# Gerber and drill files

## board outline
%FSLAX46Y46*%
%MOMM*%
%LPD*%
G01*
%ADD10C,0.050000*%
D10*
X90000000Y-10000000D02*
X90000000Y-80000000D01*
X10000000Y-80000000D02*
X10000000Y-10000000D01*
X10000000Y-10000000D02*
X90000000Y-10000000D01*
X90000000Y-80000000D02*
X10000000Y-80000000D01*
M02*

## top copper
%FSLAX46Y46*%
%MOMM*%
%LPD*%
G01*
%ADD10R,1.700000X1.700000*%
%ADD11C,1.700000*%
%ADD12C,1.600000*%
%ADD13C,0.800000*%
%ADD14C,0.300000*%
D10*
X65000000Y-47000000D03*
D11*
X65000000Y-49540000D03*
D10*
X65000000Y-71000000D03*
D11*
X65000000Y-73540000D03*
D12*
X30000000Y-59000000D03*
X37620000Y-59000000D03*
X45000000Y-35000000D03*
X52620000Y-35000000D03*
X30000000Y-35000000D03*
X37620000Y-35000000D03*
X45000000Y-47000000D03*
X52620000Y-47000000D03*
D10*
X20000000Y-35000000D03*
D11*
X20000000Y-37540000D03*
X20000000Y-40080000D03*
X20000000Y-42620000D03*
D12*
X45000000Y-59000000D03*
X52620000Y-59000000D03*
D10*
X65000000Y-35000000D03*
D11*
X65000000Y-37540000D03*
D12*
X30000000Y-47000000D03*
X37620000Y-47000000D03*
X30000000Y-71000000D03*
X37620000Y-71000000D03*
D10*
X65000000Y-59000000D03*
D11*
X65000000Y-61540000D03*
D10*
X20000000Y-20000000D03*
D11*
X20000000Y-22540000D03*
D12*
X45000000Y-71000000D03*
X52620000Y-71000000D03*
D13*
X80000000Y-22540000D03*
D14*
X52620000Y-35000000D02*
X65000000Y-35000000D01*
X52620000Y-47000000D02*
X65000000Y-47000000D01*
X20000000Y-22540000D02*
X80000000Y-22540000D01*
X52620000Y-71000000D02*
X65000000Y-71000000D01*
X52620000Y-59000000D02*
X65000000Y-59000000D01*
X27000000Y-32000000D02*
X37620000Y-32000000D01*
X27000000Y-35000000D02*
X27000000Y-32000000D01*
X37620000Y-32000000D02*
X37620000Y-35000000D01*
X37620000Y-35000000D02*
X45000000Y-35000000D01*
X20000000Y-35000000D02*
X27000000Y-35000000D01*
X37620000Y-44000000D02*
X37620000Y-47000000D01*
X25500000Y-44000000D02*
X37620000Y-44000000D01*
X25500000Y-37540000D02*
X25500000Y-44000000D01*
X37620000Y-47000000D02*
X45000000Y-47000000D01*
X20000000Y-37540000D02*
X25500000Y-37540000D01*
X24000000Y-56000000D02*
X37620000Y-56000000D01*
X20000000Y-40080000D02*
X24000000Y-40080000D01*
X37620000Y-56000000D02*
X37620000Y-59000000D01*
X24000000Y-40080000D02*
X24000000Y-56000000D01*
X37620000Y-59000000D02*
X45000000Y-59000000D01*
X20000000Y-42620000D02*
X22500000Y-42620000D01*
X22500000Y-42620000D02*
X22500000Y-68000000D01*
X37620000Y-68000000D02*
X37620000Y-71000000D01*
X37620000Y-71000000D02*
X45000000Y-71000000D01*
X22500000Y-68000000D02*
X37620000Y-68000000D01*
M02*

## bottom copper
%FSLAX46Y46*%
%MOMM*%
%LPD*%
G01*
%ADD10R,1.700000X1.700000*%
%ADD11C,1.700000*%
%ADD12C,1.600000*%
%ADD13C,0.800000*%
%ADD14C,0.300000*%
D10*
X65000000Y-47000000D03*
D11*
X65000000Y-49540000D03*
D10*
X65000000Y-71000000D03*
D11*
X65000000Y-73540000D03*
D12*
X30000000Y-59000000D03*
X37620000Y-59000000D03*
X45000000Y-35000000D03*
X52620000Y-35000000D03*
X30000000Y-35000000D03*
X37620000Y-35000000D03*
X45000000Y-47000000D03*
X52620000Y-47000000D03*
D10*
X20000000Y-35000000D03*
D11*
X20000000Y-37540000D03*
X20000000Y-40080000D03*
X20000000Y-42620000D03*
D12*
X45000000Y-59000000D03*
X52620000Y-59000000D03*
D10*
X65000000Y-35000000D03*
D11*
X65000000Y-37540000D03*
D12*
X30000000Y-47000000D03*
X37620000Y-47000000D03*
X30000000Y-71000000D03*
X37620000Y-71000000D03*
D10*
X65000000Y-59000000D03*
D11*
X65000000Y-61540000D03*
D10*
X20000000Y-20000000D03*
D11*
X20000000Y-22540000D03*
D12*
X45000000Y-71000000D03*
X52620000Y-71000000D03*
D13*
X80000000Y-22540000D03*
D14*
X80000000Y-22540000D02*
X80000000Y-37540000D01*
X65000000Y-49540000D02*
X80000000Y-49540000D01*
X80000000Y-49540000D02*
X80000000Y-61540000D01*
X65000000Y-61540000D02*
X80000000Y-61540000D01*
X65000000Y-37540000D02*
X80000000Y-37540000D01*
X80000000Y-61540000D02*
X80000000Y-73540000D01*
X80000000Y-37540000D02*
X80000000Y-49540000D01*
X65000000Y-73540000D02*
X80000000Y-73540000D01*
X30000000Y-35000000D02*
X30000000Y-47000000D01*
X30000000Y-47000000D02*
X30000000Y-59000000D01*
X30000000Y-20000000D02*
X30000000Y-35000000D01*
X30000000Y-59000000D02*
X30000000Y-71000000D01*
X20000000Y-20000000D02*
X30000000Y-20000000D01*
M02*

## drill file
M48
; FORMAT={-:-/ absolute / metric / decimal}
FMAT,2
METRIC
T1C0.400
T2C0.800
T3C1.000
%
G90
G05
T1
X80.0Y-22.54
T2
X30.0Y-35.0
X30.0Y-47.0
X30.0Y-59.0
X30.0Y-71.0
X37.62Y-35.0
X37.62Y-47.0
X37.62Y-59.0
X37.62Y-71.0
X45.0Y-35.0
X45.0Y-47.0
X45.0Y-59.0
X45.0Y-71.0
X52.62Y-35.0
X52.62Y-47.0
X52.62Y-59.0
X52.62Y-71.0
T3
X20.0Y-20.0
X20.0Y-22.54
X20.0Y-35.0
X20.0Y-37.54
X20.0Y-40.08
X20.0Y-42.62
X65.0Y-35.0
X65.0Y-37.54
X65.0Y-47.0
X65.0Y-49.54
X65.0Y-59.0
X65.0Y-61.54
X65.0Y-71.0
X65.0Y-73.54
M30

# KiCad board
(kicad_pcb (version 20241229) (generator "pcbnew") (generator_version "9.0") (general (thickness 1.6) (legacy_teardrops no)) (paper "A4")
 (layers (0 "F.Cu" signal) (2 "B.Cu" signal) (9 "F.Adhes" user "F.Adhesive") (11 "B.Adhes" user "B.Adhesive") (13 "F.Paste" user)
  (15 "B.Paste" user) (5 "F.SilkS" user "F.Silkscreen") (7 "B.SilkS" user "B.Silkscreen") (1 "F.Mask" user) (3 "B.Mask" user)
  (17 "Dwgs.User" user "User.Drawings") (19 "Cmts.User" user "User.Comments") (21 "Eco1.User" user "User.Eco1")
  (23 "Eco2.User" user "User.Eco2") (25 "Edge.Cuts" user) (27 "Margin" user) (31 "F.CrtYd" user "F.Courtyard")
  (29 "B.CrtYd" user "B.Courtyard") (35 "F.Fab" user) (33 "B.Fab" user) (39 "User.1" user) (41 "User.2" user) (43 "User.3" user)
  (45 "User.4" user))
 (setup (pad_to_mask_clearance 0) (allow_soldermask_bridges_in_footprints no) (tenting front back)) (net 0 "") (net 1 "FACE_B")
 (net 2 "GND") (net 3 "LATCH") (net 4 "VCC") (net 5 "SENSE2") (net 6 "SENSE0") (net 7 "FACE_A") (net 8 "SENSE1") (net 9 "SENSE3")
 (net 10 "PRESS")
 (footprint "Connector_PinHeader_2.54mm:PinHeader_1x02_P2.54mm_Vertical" (layer "F.Cu") (at 65 47)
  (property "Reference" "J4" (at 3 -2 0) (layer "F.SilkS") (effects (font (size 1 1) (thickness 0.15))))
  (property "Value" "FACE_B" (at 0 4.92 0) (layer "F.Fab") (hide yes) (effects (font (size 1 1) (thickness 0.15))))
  (pad "1" thru_hole rect (at 0 0) (size 1.7 1.7) (drill 1) (layers "*.Cu" "*.Mask") (remove_unused_layers no) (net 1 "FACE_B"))
  (pad "2" thru_hole circle (at 0 2.54) (size 1.7 1.7) (drill 1) (layers "*.Cu" "*.Mask") (remove_unused_layers no) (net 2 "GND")))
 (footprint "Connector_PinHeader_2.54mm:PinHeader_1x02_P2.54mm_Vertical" (layer "F.Cu") (at 65 71)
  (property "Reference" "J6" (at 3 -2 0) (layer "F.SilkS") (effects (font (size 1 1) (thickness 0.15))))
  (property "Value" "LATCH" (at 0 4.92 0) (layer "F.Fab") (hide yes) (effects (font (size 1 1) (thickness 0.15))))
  (pad "1" thru_hole rect (at 0 0) (size 1.7 1.7) (drill 1) (layers "*.Cu" "*.Mask") (remove_unused_layers no) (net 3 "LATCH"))
  (pad "2" thru_hole circle (at 0 2.54) (size 1.7 1.7) (drill 1) (layers "*.Cu" "*.Mask") (remove_unused_layers no) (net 2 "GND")))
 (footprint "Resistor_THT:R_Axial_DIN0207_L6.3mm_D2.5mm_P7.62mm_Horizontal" (layer "F.Cu") (at 30 59)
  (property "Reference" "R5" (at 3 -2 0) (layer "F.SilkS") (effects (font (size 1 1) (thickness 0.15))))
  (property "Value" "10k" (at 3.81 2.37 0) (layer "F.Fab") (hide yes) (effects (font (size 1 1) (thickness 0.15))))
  (pad "1" thru_hole circle (at 0 0) (size 1.6 1.6) (drill 0.8) (layers "*.Cu" "*.Mask") (remove_unused_layers no) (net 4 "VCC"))
  (pad "2" thru_hole circle (at 7.62 0) (size 1.6 1.6) (drill 0.8) (layers "*.Cu" "*.Mask") (remove_unused_layers no) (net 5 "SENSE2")))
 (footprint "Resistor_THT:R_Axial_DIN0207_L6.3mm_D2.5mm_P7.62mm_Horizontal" (layer "F.Cu") (at 45 35)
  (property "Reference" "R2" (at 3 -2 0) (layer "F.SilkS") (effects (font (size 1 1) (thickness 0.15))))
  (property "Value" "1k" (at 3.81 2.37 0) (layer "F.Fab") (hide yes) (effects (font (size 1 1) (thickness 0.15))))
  (pad "1" thru_hole circle (at 0 0) (size 1.6 1.6) (drill 0.8) (layers "*.Cu" "*.Mask") (remove_unused_layers no) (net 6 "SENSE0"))
  (pad "2" thru_hole circle (at 7.62 0) (size 1.6 1.6) (drill 0.8) (layers "*.Cu" "*.Mask") (remove_unused_layers no) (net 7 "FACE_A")))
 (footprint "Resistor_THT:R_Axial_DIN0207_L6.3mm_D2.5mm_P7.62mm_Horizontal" (layer "F.Cu") (at 30 35)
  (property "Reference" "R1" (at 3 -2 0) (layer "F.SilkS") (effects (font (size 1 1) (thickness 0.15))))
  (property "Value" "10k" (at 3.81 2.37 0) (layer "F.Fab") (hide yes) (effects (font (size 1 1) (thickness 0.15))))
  (pad "1" thru_hole circle (at 0 0) (size 1.6 1.6) (drill 0.8) (layers "*.Cu" "*.Mask") (remove_unused_layers no) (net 4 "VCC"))
  (pad "2" thru_hole circle (at 7.62 0) (size 1.6 1.6) (drill 0.8) (layers "*.Cu" "*.Mask") (remove_unused_layers no) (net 6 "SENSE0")))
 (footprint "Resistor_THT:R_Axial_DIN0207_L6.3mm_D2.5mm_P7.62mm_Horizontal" (layer "F.Cu") (at 45 47)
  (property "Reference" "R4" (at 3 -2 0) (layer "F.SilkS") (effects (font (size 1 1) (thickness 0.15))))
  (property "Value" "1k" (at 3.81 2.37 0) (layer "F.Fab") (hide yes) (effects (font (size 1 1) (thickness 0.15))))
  (pad "1" thru_hole circle (at 0 0) (size 1.6 1.6) (drill 0.8) (layers "*.Cu" "*.Mask") (remove_unused_layers no) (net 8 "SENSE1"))
  (pad "2" thru_hole circle (at 7.62 0) (size 1.6 1.6) (drill 0.8) (layers "*.Cu" "*.Mask") (remove_unused_layers no) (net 1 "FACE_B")))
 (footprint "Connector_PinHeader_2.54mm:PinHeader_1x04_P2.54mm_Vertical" (layer "F.Cu") (at 20 35)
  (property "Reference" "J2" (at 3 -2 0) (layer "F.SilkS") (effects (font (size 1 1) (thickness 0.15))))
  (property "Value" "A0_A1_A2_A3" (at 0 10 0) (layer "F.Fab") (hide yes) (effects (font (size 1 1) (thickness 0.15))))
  (pad "1" thru_hole rect (at 0 0) (size 1.7 1.7) (drill 1) (layers "*.Cu" "*.Mask") (remove_unused_layers no) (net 6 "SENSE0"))
  (pad "2" thru_hole circle (at 0 2.54) (size 1.7 1.7) (drill 1) (layers "*.Cu" "*.Mask") (remove_unused_layers no) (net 8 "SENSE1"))
  (pad "3" thru_hole circle (at 0 5.08) (size 1.7 1.7) (drill 1) (layers "*.Cu" "*.Mask") (remove_unused_layers no) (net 5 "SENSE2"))
  (pad "4" thru_hole circle (at 0 7.62) (size 1.7 1.7) (drill 1) (layers "*.Cu" "*.Mask") (remove_unused_layers no) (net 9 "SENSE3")))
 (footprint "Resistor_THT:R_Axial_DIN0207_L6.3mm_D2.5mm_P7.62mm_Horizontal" (layer "F.Cu") (at 45 59)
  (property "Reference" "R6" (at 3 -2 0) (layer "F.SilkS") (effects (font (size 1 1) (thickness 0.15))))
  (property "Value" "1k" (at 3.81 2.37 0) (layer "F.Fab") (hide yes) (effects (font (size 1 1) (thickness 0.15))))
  (pad "1" thru_hole circle (at 0 0) (size 1.6 1.6) (drill 0.8) (layers "*.Cu" "*.Mask") (remove_unused_layers no) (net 5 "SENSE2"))
  (pad "2" thru_hole circle (at 7.62 0) (size 1.6 1.6) (drill 0.8) (layers "*.Cu" "*.Mask") (remove_unused_layers no) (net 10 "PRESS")))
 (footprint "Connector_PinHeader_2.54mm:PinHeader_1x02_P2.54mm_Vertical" (layer "F.Cu") (at 65 35)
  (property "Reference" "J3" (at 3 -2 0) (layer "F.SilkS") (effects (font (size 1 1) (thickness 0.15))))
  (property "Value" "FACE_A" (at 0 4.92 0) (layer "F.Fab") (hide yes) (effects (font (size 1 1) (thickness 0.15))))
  (pad "1" thru_hole rect (at 0 0) (size 1.7 1.7) (drill 1) (layers "*.Cu" "*.Mask") (remove_unused_layers no) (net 7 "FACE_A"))
  (pad "2" thru_hole circle (at 0 2.54) (size 1.7 1.7) (drill 1) (layers "*.Cu" "*.Mask") (remove_unused_layers no) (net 2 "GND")))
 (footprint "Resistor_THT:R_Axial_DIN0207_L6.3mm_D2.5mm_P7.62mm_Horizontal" (layer "F.Cu") (at 30 47)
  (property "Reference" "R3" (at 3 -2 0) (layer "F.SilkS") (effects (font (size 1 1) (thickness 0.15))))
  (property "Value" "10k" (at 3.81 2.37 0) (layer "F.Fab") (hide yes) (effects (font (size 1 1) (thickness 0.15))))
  (pad "1" thru_hole circle (at 0 0) (size 1.6 1.6) (drill 0.8) (layers "*.Cu" "*.Mask") (remove_unused_layers no) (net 4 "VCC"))
  (pad "2" thru_hole circle (at 7.62 0) (size 1.6 1.6) (drill 0.8) (layers "*.Cu" "*.Mask") (remove_unused_layers no) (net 8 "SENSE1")))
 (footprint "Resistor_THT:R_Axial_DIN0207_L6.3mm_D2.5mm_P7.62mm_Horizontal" (layer "F.Cu") (at 30 71)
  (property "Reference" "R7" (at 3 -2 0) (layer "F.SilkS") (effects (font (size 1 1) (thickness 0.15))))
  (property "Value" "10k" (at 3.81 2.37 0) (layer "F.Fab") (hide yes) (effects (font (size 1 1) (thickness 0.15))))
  (pad "1" thru_hole circle (at 0 0) (size 1.6 1.6) (drill 0.8) (layers "*.Cu" "*.Mask") (remove_unused_layers no) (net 4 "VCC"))
  (pad "2" thru_hole circle (at 7.62 0) (size 1.6 1.6) (drill 0.8) (layers "*.Cu" "*.Mask") (remove_unused_layers no) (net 9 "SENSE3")))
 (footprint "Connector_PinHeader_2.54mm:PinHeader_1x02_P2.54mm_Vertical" (layer "F.Cu") (at 65 59)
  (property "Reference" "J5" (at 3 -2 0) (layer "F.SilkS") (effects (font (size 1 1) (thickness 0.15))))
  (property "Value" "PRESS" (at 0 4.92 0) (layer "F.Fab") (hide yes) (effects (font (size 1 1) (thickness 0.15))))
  (pad "1" thru_hole rect (at 0 0) (size 1.7 1.7) (drill 1) (layers "*.Cu" "*.Mask") (remove_unused_layers no) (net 10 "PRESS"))
  (pad "2" thru_hole circle (at 0 2.54) (size 1.7 1.7) (drill 1) (layers "*.Cu" "*.Mask") (remove_unused_layers no) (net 2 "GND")))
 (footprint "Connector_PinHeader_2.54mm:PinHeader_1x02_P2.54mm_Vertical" (layer "F.Cu") (at 20 20)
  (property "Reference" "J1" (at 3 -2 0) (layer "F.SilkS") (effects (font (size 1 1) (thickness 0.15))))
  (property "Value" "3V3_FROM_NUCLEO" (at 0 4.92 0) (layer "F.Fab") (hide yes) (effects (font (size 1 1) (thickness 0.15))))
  (pad "1" thru_hole rect (at 0 0) (size 1.7 1.7) (drill 1) (layers "*.Cu" "*.Mask") (remove_unused_layers no) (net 4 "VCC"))
  (pad "2" thru_hole circle (at 0 2.54) (size 1.7 1.7) (drill 1) (layers "*.Cu" "*.Mask") (remove_unused_layers no) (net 2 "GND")))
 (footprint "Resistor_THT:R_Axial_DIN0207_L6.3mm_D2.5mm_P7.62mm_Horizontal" (layer "F.Cu") (at 45 71)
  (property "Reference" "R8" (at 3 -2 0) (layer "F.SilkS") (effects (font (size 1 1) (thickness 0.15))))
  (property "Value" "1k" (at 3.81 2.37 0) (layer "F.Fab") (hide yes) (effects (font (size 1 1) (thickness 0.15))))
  (pad "1" thru_hole circle (at 0 0) (size 1.6 1.6) (drill 0.8) (layers "*.Cu" "*.Mask") (remove_unused_layers no) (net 9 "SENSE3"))
  (pad "2" thru_hole circle (at 7.62 0) (size 1.6 1.6) (drill 0.8) (layers "*.Cu" "*.Mask") (remove_unused_layers no) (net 3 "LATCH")))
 (gr_line (start 90 10) (end 90 80) (stroke (width 0.05) (type default)) (layer "Edge.Cuts"))
 (gr_line (start 10 80) (end 10 10) (stroke (width 0.05) (type default)) (layer "Edge.Cuts"))
 (gr_line (start 10 10) (end 90 10) (stroke (width 0.05) (type default)) (layer "Edge.Cuts"))
 (gr_line (start 90 80) (end 10 80) (stroke (width 0.05) (type default)) (layer "Edge.Cuts"))
 (segment (start 52.62 35) (end 65 35) (width 0.3) (layer "F.Cu") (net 7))
 (segment (start 52.62 47) (end 65 47) (width 0.3) (layer "F.Cu") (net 1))
 (segment (start 20 22.54) (end 80 22.54) (width 0.3) (layer "F.Cu") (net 2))
 (via (at 80 22.54) (size 0.8) (drill 0.4) (layers "F.Cu" "B.Cu") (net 2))
 (segment (start 80 22.54) (end 80 37.54) (width 0.3) (layer "B.Cu") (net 2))
 (segment (start 65 49.54) (end 80 49.54) (width 0.3) (layer "B.Cu") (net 2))
 (segment (start 80 49.54) (end 80 61.54) (width 0.3) (layer "B.Cu") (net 2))
 (segment (start 65 61.54) (end 80 61.54) (width 0.3) (layer "B.Cu") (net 2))
 (segment (start 65 37.54) (end 80 37.54) (width 0.3) (layer "B.Cu") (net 2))
 (segment (start 80 61.54) (end 80 73.54) (width 0.3) (layer "B.Cu") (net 2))
 (segment (start 80 37.54) (end 80 49.54) (width 0.3) (layer "B.Cu") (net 2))
 (segment (start 65 73.54) (end 80 73.54) (width 0.3) (layer "B.Cu") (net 2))
 (segment (start 52.62 71) (end 65 71) (width 0.3) (layer "F.Cu") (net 3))
 (segment (start 52.62 59) (end 65 59) (width 0.3) (layer "F.Cu") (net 10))
 (segment (start 27 32) (end 37.62 32) (width 0.3) (layer "F.Cu") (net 6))
 (segment (start 27 35) (end 27 32) (width 0.3) (layer "F.Cu") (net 6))
 (segment (start 37.62 32) (end 37.62 35) (width 0.3) (layer "F.Cu") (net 6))
 (segment (start 37.62 35) (end 45 35) (width 0.3) (layer "F.Cu") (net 6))
 (segment (start 20 35) (end 27 35) (width 0.3) (layer "F.Cu") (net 6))
 (segment (start 37.62 44) (end 37.62 47) (width 0.3) (layer "F.Cu") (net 8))
 (segment (start 25.5 44) (end 37.62 44) (width 0.3) (layer "F.Cu") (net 8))
 (segment (start 25.5 37.54) (end 25.5 44) (width 0.3) (layer "F.Cu") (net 8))
 (segment (start 37.62 47) (end 45 47) (width 0.3) (layer "F.Cu") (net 8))
 (segment (start 20 37.54) (end 25.5 37.54) (width 0.3) (layer "F.Cu") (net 8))
 (segment (start 24 56) (end 37.62 56) (width 0.3) (layer "F.Cu") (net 5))
 (segment (start 20 40.08) (end 24 40.08) (width 0.3) (layer "F.Cu") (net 5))
 (segment (start 37.62 56) (end 37.62 59) (width 0.3) (layer "F.Cu") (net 5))
 (segment (start 24 40.08) (end 24 56) (width 0.3) (layer "F.Cu") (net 5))
 (segment (start 37.62 59) (end 45 59) (width 0.3) (layer "F.Cu") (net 5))
 (segment (start 20 42.62) (end 22.5 42.62) (width 0.3) (layer "F.Cu") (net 9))
 (segment (start 22.5 42.62) (end 22.5 68) (width 0.3) (layer "F.Cu") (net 9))
 (segment (start 37.62 68) (end 37.62 71) (width 0.3) (layer "F.Cu") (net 9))
 (segment (start 37.62 71) (end 45 71) (width 0.3) (layer "F.Cu") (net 9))
 (segment (start 22.5 68) (end 37.62 68) (width 0.3) (layer "F.Cu") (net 9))
 (segment (start 30 35) (end 30 47) (width 0.3) (layer "B.Cu") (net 4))
 (segment (start 30 47) (end 30 59) (width 0.3) (layer "B.Cu") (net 4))
 (segment (start 30 20) (end 30 35) (width 0.3) (layer "B.Cu") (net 4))
 (segment (start 30 59) (end 30 71) (width 0.3) (layer "B.Cu") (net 4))
 (segment (start 20 20) (end 30 20) (width 0.3) (layer "B.Cu") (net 4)))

